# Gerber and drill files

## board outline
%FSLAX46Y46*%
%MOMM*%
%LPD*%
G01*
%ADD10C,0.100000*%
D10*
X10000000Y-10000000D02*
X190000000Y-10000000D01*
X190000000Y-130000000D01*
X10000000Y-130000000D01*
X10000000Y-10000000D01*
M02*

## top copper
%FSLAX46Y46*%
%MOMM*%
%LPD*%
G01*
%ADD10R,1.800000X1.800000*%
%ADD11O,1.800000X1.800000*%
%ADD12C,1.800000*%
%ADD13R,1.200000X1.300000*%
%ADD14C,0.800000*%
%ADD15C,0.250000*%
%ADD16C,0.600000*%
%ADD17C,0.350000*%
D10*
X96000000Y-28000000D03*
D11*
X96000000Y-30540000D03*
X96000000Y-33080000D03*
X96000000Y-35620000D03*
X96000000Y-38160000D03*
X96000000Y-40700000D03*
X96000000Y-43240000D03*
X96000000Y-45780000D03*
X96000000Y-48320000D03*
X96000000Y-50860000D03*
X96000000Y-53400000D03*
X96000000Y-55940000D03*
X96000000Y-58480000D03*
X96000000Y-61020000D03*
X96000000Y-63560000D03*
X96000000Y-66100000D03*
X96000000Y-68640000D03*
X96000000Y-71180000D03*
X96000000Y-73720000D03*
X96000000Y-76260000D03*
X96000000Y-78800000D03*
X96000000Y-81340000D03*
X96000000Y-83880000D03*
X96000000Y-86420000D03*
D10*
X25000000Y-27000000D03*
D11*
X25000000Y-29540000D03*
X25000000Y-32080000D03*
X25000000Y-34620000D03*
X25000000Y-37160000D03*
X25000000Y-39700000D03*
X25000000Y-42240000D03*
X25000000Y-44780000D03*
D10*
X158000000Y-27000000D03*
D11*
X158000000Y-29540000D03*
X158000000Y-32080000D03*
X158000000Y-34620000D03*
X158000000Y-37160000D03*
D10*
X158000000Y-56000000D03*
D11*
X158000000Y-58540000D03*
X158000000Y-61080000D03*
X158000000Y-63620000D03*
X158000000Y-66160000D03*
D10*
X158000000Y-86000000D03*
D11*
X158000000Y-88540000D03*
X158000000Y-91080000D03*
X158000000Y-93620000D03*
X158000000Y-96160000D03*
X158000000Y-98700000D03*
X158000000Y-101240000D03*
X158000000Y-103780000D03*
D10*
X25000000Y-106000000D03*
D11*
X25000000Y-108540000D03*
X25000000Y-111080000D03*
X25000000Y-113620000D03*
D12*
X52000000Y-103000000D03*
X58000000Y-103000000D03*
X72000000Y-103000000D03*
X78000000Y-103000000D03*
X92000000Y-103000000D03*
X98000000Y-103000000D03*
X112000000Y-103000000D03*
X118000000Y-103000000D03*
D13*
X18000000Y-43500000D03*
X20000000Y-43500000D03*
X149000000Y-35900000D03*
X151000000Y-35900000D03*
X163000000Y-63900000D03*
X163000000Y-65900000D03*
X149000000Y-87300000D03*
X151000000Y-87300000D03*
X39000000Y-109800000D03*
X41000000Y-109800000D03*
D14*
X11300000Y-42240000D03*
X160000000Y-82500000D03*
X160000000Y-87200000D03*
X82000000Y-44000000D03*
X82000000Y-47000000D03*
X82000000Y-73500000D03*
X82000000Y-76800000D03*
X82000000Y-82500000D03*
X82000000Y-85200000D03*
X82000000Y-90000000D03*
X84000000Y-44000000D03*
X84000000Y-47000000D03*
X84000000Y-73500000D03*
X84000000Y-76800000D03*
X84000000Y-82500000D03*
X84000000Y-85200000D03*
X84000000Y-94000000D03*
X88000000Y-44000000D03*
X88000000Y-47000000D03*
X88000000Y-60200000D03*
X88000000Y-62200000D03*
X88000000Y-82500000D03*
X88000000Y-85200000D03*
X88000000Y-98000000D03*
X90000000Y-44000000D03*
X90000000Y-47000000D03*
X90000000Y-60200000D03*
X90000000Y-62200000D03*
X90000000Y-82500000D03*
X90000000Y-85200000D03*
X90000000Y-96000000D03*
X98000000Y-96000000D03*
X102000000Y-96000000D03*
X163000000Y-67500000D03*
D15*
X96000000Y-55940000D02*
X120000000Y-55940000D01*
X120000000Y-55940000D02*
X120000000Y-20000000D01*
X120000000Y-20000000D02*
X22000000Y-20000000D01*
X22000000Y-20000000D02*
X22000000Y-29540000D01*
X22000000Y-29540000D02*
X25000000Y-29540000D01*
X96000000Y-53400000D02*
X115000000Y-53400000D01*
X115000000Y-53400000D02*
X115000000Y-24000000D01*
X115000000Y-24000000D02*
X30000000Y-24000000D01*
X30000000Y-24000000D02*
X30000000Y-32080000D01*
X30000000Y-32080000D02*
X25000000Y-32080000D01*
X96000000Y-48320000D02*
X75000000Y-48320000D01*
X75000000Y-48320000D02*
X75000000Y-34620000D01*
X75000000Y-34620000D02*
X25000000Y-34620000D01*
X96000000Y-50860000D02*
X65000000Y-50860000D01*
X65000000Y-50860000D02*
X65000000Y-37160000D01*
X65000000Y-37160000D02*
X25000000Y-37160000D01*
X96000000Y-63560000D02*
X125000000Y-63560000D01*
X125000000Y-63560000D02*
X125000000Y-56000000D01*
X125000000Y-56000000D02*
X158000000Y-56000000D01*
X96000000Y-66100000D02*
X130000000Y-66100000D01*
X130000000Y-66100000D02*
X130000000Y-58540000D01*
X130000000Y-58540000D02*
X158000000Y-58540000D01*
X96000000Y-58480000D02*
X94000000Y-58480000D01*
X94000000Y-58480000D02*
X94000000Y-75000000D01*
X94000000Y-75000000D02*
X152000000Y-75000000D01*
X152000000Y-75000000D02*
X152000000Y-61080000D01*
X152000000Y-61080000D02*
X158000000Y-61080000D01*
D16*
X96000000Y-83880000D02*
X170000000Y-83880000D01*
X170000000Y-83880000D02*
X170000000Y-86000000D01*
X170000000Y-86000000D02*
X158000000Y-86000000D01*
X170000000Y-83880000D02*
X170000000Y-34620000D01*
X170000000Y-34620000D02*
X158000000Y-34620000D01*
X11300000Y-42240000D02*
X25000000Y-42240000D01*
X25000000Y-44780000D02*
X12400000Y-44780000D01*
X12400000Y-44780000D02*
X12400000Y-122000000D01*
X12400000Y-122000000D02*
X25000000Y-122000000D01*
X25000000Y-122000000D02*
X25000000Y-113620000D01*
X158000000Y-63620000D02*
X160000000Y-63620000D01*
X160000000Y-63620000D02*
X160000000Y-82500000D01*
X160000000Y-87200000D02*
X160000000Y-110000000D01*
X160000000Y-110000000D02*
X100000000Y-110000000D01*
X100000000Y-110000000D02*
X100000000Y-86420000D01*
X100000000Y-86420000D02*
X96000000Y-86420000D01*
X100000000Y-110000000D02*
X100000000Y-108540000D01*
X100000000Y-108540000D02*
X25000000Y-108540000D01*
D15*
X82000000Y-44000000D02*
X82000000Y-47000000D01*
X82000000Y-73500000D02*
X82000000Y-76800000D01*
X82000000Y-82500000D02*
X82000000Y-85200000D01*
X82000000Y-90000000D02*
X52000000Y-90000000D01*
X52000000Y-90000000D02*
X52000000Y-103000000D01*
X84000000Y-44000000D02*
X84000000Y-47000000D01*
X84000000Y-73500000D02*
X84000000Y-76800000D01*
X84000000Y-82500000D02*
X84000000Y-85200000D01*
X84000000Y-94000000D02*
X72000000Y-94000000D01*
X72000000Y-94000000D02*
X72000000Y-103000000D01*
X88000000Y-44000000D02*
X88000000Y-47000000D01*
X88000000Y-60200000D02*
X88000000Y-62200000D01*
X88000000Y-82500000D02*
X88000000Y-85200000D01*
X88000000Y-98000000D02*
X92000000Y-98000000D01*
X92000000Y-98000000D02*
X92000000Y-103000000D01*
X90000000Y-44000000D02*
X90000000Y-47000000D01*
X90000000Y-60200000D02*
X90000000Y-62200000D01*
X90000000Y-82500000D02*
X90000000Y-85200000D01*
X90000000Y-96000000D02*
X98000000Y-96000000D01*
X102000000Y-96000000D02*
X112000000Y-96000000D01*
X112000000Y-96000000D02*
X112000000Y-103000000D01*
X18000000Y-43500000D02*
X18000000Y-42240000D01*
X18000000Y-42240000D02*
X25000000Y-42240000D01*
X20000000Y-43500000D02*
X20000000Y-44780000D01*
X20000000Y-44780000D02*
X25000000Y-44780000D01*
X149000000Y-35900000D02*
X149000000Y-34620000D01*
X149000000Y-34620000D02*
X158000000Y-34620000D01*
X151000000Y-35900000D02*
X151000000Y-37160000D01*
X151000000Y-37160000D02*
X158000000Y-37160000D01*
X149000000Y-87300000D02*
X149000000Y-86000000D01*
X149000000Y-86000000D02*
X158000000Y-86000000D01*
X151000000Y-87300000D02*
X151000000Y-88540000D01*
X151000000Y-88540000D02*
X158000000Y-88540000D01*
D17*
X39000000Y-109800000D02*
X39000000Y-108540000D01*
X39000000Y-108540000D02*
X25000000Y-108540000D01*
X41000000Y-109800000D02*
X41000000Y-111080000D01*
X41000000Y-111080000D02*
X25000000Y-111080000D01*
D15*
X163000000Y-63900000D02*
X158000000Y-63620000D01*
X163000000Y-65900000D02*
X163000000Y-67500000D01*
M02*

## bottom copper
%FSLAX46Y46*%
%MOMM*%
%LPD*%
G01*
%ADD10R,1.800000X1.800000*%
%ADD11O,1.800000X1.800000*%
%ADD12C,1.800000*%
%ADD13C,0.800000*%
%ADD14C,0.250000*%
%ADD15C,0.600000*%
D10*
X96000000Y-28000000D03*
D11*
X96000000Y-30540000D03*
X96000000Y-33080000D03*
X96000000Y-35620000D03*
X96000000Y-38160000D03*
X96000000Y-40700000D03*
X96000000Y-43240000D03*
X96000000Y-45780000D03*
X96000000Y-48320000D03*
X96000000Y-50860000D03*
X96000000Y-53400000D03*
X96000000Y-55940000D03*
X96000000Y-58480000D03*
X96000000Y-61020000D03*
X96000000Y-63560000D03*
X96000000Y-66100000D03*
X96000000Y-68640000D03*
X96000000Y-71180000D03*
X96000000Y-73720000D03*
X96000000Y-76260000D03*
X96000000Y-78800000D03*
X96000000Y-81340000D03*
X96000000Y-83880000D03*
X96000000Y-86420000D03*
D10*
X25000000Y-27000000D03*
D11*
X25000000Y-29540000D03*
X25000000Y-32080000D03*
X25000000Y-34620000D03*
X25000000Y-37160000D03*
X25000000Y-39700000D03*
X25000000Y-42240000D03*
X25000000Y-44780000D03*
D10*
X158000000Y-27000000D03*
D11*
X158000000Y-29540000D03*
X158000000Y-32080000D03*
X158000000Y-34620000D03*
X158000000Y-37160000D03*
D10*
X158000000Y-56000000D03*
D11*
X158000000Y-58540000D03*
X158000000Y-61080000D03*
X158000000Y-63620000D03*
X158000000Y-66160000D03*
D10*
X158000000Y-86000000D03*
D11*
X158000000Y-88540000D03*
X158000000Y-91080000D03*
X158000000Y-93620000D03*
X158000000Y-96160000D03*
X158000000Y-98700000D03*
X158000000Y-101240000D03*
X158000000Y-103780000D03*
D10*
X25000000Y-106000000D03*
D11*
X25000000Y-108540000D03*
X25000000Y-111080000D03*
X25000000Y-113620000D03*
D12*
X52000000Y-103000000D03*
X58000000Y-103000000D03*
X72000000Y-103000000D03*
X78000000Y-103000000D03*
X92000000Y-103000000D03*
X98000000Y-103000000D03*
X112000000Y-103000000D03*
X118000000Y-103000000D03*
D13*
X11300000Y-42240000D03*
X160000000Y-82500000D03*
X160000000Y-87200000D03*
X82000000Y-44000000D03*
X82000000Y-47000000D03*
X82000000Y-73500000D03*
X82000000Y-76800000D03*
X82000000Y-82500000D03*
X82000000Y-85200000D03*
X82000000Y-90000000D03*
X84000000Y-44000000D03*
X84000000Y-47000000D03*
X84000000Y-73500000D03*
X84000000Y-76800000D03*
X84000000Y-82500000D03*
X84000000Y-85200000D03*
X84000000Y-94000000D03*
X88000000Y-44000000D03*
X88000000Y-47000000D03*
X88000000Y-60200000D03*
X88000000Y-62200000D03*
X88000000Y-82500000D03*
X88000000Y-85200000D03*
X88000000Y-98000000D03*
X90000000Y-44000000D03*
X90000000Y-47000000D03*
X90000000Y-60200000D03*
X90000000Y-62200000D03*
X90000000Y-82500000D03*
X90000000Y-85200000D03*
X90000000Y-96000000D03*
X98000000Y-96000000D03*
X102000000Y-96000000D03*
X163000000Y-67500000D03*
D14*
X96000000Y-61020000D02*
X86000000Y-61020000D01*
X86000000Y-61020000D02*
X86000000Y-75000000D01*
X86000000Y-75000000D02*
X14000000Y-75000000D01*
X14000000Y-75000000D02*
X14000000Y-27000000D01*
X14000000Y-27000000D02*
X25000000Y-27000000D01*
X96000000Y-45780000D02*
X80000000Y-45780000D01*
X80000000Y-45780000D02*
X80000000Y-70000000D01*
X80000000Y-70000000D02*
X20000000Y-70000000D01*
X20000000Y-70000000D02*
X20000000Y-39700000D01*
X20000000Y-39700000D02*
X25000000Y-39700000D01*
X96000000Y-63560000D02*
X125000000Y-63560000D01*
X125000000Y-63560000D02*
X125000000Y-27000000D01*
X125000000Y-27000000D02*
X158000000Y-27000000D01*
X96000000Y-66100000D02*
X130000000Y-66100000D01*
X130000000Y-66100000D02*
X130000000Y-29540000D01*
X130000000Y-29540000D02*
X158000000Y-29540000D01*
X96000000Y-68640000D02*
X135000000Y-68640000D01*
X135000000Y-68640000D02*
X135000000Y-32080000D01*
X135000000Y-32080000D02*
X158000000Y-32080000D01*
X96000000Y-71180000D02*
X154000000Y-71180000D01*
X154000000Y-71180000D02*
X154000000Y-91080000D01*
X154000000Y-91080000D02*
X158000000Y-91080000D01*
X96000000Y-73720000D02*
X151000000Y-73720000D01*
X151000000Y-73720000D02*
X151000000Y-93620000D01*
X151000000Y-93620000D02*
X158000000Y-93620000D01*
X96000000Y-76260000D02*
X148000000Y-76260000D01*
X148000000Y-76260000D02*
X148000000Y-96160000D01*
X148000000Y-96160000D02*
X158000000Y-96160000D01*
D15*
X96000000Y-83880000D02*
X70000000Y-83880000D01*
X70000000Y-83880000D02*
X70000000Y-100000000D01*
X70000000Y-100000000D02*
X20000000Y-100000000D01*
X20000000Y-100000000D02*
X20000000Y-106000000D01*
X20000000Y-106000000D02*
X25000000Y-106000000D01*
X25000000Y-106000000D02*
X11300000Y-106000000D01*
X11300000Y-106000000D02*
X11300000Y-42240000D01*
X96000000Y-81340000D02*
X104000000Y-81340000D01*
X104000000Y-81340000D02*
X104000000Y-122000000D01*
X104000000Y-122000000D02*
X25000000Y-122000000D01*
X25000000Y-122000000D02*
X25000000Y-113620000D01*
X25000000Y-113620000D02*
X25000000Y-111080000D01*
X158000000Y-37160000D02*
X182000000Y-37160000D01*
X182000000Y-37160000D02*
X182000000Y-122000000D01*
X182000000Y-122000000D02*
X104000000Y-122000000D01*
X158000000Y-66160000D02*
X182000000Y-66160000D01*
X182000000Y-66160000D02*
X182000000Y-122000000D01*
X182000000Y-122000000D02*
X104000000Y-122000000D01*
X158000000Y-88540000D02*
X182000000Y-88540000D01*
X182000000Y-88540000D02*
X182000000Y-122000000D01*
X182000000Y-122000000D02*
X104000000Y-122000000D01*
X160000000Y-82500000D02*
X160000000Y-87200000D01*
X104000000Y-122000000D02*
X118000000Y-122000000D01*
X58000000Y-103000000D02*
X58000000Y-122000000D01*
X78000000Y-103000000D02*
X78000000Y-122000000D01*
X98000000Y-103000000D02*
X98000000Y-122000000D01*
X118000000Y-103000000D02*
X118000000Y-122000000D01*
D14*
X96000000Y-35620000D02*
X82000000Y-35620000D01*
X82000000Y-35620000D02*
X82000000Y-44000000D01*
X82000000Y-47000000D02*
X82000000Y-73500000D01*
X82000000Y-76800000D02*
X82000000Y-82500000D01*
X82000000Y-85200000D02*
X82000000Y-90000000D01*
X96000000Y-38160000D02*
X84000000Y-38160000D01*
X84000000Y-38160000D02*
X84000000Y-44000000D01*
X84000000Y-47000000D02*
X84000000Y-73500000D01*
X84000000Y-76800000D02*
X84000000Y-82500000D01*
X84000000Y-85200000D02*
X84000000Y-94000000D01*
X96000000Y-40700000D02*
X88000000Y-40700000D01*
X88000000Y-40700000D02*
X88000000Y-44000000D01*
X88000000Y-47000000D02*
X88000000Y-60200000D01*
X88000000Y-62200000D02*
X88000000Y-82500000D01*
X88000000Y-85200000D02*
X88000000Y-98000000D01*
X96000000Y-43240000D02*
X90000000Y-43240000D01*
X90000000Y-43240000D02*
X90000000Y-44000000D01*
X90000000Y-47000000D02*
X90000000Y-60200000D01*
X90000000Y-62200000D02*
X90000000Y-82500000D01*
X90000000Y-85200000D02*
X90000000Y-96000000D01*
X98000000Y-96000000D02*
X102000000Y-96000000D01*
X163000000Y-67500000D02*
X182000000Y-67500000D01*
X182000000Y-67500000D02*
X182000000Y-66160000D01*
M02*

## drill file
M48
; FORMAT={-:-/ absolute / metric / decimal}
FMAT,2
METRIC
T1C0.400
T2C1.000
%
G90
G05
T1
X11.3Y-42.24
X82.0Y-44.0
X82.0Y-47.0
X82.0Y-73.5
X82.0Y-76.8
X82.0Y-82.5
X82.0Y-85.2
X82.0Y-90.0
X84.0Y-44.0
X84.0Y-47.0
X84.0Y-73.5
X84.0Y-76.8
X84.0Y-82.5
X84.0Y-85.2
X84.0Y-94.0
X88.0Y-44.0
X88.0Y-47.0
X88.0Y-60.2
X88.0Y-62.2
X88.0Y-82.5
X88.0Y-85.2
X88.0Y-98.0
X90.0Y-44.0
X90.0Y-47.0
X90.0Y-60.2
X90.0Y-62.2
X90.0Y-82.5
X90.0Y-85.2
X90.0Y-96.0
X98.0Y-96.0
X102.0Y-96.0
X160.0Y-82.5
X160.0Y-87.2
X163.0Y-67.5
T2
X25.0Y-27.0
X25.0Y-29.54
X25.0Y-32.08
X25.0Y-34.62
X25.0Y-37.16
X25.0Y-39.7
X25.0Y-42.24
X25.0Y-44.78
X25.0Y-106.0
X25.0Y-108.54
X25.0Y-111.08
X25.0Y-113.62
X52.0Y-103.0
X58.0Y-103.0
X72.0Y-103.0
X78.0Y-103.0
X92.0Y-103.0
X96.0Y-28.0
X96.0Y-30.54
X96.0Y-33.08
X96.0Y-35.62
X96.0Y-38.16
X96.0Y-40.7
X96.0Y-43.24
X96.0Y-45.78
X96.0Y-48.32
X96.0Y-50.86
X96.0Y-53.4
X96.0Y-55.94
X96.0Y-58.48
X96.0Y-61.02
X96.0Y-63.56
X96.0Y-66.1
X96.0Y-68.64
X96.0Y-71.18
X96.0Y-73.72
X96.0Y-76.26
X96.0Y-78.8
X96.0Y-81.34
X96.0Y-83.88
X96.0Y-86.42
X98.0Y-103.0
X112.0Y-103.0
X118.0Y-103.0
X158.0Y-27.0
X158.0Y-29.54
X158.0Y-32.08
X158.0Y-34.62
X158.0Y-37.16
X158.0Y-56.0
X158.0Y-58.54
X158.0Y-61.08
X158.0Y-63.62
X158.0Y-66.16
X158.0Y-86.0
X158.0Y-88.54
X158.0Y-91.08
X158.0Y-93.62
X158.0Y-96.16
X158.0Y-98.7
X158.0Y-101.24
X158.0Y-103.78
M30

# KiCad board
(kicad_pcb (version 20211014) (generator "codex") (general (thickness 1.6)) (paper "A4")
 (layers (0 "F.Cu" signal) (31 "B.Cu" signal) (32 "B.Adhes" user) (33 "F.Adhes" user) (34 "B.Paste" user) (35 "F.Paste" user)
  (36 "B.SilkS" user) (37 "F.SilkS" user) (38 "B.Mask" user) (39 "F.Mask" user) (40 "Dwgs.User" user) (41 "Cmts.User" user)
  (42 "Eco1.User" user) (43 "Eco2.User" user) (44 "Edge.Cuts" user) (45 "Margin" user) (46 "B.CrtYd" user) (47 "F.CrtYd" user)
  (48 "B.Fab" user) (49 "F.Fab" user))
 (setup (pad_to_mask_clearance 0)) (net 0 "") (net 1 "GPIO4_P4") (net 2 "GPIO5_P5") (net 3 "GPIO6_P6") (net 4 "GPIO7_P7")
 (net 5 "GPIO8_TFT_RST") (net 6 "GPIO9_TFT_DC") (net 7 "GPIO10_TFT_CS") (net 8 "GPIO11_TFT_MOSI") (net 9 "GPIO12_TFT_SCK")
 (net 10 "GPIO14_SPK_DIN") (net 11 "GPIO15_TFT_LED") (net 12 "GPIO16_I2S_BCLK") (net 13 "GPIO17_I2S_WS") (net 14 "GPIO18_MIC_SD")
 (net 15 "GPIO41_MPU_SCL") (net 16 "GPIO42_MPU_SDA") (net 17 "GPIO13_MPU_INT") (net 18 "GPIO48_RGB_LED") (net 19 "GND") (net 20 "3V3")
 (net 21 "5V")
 (gr_rect (start 10 10) (end 190 130) (layer "Edge.Cuts") (width 0.1))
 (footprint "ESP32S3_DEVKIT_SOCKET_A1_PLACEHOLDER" (layer "F.Cu") (at 96 28)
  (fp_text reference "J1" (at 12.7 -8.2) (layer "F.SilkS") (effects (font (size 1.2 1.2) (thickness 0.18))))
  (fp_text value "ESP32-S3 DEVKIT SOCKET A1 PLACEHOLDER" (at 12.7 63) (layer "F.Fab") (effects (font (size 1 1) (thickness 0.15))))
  (pad "1" thru_hole rect (at 0 0) (size 1.8 1.8) (drill 1) (layers *.Cu *.Mask))
  (pad "2" thru_hole oval (at 0 2.54) (size 1.8 1.8) (drill 1) (layers *.Cu *.Mask))
  (pad "3" thru_hole oval (at 0 5.08) (size 1.8 1.8) (drill 1) (layers *.Cu *.Mask))
  (pad "4" thru_hole oval (at 0 7.62) (size 1.8 1.8) (drill 1) (layers *.Cu *.Mask) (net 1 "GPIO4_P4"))
  (pad "5" thru_hole oval (at 0 10.16) (size 1.8 1.8) (drill 1) (layers *.Cu *.Mask) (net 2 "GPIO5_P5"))
  (pad "6" thru_hole oval (at 0 12.7) (size 1.8 1.8) (drill 1) (layers *.Cu *.Mask) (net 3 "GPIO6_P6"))
  (pad "7" thru_hole oval (at 0 15.24) (size 1.8 1.8) (drill 1) (layers *.Cu *.Mask) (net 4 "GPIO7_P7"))
  (pad "8" thru_hole oval (at 0 17.78) (size 1.8 1.8) (drill 1) (layers *.Cu *.Mask) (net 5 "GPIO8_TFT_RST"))
  (pad "9" thru_hole oval (at 0 20.32) (size 1.8 1.8) (drill 1) (layers *.Cu *.Mask) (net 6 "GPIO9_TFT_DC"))
  (pad "10" thru_hole oval (at 0 22.86) (size 1.8 1.8) (drill 1) (layers *.Cu *.Mask) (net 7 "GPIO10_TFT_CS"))
  (pad "11" thru_hole oval (at 0 25.4) (size 1.8 1.8) (drill 1) (layers *.Cu *.Mask) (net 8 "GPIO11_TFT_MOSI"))
  (pad "12" thru_hole oval (at 0 27.94) (size 1.8 1.8) (drill 1) (layers *.Cu *.Mask) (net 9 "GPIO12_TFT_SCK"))
  (pad "13" thru_hole oval (at 0 30.48) (size 1.8 1.8) (drill 1) (layers *.Cu *.Mask) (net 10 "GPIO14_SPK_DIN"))
  (pad "14" thru_hole oval (at 0 33.02) (size 1.8 1.8) (drill 1) (layers *.Cu *.Mask) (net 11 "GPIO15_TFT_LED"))
  (pad "15" thru_hole oval (at 0 35.56) (size 1.8 1.8) (drill 1) (layers *.Cu *.Mask) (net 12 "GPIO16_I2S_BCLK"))
  (pad "16" thru_hole oval (at 0 38.1) (size 1.8 1.8) (drill 1) (layers *.Cu *.Mask) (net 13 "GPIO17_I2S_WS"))
  (pad "17" thru_hole oval (at 0 40.64) (size 1.8 1.8) (drill 1) (layers *.Cu *.Mask) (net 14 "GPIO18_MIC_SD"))
  (pad "18" thru_hole oval (at 0 43.18) (size 1.8 1.8) (drill 1) (layers *.Cu *.Mask) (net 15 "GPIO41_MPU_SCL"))
  (pad "19" thru_hole oval (at 0 45.72) (size 1.8 1.8) (drill 1) (layers *.Cu *.Mask) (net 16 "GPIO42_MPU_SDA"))
  (pad "20" thru_hole oval (at 0 48.26) (size 1.8 1.8) (drill 1) (layers *.Cu *.Mask) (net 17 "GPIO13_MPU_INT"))
  (pad "21" thru_hole oval (at 0 50.8) (size 1.8 1.8) (drill 1) (layers *.Cu *.Mask) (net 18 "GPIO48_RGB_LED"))
  (pad "22" thru_hole oval (at 0 53.34) (size 1.8 1.8) (drill 1) (layers *.Cu *.Mask) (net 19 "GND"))
  (pad "23" thru_hole oval (at 0 55.88) (size 1.8 1.8) (drill 1) (layers *.Cu *.Mask) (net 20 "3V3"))
  (pad "24" thru_hole oval (at 0 58.42) (size 1.8 1.8) (drill 1) (layers *.Cu *.Mask) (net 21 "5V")))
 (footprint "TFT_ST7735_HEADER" (layer "F.Cu") (at 25 27)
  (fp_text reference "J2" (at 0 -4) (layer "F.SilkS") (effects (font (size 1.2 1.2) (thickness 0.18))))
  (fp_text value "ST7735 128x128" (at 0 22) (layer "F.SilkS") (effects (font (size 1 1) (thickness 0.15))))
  (pad "1" thru_hole rect (at 0 0) (size 1.8 1.8) (drill 1) (layers *.Cu *.Mask) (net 11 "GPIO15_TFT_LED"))
  (pad "2" thru_hole oval (at 0 2.54) (size 1.8 1.8) (drill 1) (layers *.Cu *.Mask) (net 9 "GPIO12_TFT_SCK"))
  (pad "3" thru_hole oval (at 0 5.08) (size 1.8 1.8) (drill 1) (layers *.Cu *.Mask) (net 8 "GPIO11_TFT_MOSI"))
  (pad "4" thru_hole oval (at 0 7.62) (size 1.8 1.8) (drill 1) (layers *.Cu *.Mask) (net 6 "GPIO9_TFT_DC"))
  (pad "5" thru_hole oval (at 0 10.16) (size 1.8 1.8) (drill 1) (layers *.Cu *.Mask) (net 7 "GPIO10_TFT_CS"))
  (pad "6" thru_hole oval (at 0 12.7) (size 1.8 1.8) (drill 1) (layers *.Cu *.Mask) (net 5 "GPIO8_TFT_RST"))
  (pad "7" thru_hole oval (at 0 15.24) (size 1.8 1.8) (drill 1) (layers *.Cu *.Mask) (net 20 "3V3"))
  (pad "8" thru_hole oval (at 0 17.78) (size 1.8 1.8) (drill 1) (layers *.Cu *.Mask) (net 19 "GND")))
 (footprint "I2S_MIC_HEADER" (layer "F.Cu") (at 158 27)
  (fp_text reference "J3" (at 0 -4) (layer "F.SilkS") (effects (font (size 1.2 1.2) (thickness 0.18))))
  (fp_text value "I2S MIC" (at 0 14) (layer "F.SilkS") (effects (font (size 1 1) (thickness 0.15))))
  (pad "1" thru_hole rect (at 0 0) (size 1.8 1.8) (drill 1) (layers *.Cu *.Mask) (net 12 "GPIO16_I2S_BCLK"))
  (pad "2" thru_hole oval (at 0 2.54) (size 1.8 1.8) (drill 1) (layers *.Cu *.Mask) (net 13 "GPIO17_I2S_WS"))
  (pad "3" thru_hole oval (at 0 5.08) (size 1.8 1.8) (drill 1) (layers *.Cu *.Mask) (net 14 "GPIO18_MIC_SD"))
  (pad "4" thru_hole oval (at 0 7.62) (size 1.8 1.8) (drill 1) (layers *.Cu *.Mask) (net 20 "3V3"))
  (pad "5" thru_hole oval (at 0 10.16) (size 1.8 1.8) (drill 1) (layers *.Cu *.Mask) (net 19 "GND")))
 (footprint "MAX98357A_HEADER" (layer "F.Cu") (at 158 56)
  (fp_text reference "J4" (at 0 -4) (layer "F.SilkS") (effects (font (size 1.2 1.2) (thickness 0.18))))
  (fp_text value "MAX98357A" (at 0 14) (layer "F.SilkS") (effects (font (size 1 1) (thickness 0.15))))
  (pad "1" thru_hole rect (at 0 0) (size 1.8 1.8) (drill 1) (layers *.Cu *.Mask) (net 12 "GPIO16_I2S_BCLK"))
  (pad "2" thru_hole oval (at 0 2.54) (size 1.8 1.8) (drill 1) (layers *.Cu *.Mask) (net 13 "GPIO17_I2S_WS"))
  (pad "3" thru_hole oval (at 0 5.08) (size 1.8 1.8) (drill 1) (layers *.Cu *.Mask) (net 10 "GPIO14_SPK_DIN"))
  (pad "4" thru_hole oval (at 0 7.62) (size 1.8 1.8) (drill 1) (layers *.Cu *.Mask) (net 21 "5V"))
  (pad "5" thru_hole oval (at 0 10.16) (size 1.8 1.8) (drill 1) (layers *.Cu *.Mask) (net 19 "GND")))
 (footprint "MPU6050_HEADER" (layer "F.Cu") (at 158 86)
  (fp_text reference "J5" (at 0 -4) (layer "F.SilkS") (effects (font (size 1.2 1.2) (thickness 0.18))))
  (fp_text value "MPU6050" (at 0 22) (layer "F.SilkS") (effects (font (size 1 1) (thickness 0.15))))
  (pad "1" thru_hole rect (at 0 0) (size 1.8 1.8) (drill 1) (layers *.Cu *.Mask) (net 20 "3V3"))
  (pad "2" thru_hole oval (at 0 2.54) (size 1.8 1.8) (drill 1) (layers *.Cu *.Mask) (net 19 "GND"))
  (pad "3" thru_hole oval (at 0 5.08) (size 1.8 1.8) (drill 1) (layers *.Cu *.Mask) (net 15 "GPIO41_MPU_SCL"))
  (pad "4" thru_hole oval (at 0 7.62) (size 1.8 1.8) (drill 1) (layers *.Cu *.Mask) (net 16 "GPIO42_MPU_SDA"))
  (pad "5" thru_hole oval (at 0 10.16) (size 1.8 1.8) (drill 1) (layers *.Cu *.Mask) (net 17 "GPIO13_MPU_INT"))
  (pad "6" thru_hole oval (at 0 12.7) (size 1.8 1.8) (drill 1) (layers *.Cu *.Mask))
  (pad "7" thru_hole oval (at 0 15.24) (size 1.8 1.8) (drill 1) (layers *.Cu *.Mask))
  (pad "8" thru_hole oval (at 0 17.78) (size 1.8 1.8) (drill 1) (layers *.Cu *.Mask)))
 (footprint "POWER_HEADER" (layer "F.Cu") (at 25 106)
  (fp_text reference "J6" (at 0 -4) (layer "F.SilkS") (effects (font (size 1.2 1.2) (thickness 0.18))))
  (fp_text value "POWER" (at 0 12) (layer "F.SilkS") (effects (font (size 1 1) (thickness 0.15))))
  (pad "1" thru_hole rect (at 0 0) (size 1.8 1.8) (drill 1) (layers *.Cu *.Mask) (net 20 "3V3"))
  (pad "2" thru_hole oval (at 0 2.54) (size 1.8 1.8) (drill 1) (layers *.Cu *.Mask) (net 21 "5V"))
  (pad "3" thru_hole oval (at 0 5.08) (size 1.8 1.8) (drill 1) (layers *.Cu *.Mask) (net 19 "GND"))
  (pad "4" thru_hole oval (at 0 7.62) (size 1.8 1.8) (drill 1) (layers *.Cu *.Mask) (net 19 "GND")))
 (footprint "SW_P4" (layer "F.Cu") (at 55 103)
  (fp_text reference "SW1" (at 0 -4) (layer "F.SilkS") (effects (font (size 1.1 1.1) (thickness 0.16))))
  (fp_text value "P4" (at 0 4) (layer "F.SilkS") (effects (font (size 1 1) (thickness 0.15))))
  (pad "1" thru_hole circle (at -3 0) (size 1.8 1.8) (drill 1) (layers *.Cu *.Mask) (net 1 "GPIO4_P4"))
  (pad "2" thru_hole circle (at 3 0) (size 1.8 1.8) (drill 1) (layers *.Cu *.Mask) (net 19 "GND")))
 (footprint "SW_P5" (layer "F.Cu") (at 75 103)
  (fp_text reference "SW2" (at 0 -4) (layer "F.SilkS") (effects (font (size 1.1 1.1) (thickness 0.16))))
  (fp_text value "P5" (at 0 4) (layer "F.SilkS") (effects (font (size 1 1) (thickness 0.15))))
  (pad "1" thru_hole circle (at -3 0) (size 1.8 1.8) (drill 1) (layers *.Cu *.Mask) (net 2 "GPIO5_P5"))
  (pad "2" thru_hole circle (at 3 0) (size 1.8 1.8) (drill 1) (layers *.Cu *.Mask) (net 19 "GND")))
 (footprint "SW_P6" (layer "F.Cu") (at 95 103)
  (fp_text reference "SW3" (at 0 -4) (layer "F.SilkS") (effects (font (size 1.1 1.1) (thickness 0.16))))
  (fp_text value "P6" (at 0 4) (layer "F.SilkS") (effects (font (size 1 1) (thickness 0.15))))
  (pad "1" thru_hole circle (at -3 0) (size 1.8 1.8) (drill 1) (layers *.Cu *.Mask) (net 3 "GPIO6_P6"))
  (pad "2" thru_hole circle (at 3 0) (size 1.8 1.8) (drill 1) (layers *.Cu *.Mask) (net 19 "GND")))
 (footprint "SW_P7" (layer "F.Cu") (at 115 103)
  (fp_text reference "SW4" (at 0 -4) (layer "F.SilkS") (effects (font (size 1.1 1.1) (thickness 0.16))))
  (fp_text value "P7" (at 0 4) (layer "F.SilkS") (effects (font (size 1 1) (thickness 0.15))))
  (pad "1" thru_hole circle (at -3 0) (size 1.8 1.8) (drill 1) (layers *.Cu *.Mask) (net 4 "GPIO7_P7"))
  (pad "2" thru_hole circle (at 3 0) (size 1.8 1.8) (drill 1) (layers *.Cu *.Mask) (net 19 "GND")))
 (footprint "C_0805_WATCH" (layer "F.Cu") (at 19.00 43.50)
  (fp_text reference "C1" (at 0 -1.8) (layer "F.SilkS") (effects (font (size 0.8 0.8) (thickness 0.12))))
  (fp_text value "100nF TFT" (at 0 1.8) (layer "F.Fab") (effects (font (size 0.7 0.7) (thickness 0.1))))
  (pad "1" smd rect (at -1.00 0) (size 1.20 1.30) (layers "F.Cu" "F.Paste" "F.Mask") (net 20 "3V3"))
  (pad "2" smd rect (at 1.00 0) (size 1.20 1.30) (layers "F.Cu" "F.Paste" "F.Mask") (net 19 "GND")))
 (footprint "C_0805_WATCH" (layer "F.Cu") (at 150.00 35.90)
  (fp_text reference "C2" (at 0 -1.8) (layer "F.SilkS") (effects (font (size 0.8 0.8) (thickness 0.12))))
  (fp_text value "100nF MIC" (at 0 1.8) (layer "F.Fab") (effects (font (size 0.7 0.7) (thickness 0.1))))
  (pad "1" smd rect (at -1.00 0) (size 1.20 1.30) (layers "F.Cu" "F.Paste" "F.Mask") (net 20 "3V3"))
  (pad "2" smd rect (at 1.00 0) (size 1.20 1.30) (layers "F.Cu" "F.Paste" "F.Mask") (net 19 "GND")))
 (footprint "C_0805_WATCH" (layer "F.Cu") (at 163.00 64.90 270)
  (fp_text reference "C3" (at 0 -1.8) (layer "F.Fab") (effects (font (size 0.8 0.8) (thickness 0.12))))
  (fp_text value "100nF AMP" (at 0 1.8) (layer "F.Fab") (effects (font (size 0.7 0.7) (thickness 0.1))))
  (pad "1" smd rect (at -1.00 0) (size 1.20 1.30) (layers "F.Cu" "F.Paste" "F.Mask") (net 21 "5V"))
  (pad "2" smd rect (at 1.00 0) (size 1.20 1.30) (layers "F.Cu" "F.Paste" "F.Mask") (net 19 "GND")))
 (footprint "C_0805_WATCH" (layer "F.Cu") (at 150.00 87.30)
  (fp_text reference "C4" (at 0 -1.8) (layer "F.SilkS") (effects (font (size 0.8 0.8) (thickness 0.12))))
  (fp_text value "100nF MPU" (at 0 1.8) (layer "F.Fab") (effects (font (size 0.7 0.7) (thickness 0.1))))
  (pad "1" smd rect (at -1.00 0) (size 1.20 1.30) (layers "F.Cu" "F.Paste" "F.Mask") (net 20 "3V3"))
  (pad "2" smd rect (at 1.00 0) (size 1.20 1.30) (layers "F.Cu" "F.Paste" "F.Mask") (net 19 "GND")))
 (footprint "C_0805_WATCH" (layer "F.Cu") (at 40.00 109.80)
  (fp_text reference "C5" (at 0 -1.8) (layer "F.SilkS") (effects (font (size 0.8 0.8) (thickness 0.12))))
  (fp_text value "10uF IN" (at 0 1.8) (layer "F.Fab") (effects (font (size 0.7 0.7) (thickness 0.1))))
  (pad "1" smd rect (at -1.00 0) (size 1.20 1.30) (layers "F.Cu" "F.Paste" "F.Mask") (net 21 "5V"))
  (pad "2" smd rect (at 1.00 0) (size 1.20 1.30) (layers "F.Cu" "F.Paste" "F.Mask") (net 19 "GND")))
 (segment (start 96.00 61.02) (end 86.00 61.02) (width 0.25) (layer "B.Cu") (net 11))
 (segment (start 86.00 61.02) (end 86.00 75.00) (width 0.25) (layer "B.Cu") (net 11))
 (segment (start 86.00 75.00) (end 14.00 75.00) (width 0.25) (layer "B.Cu") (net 11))
 (segment (start 14.00 75.00) (end 14.00 27.00) (width 0.25) (layer "B.Cu") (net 11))
 (segment (start 14.00 27.00) (end 25.00 27.00) (width 0.25) (layer "B.Cu") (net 11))
 (segment (start 96.00 55.94) (end 120.00 55.94) (width 0.25) (layer "F.Cu") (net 9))
 (segment (start 120.00 55.94) (end 120.00 20.00) (width 0.25) (layer "F.Cu") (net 9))
 (segment (start 120.00 20.00) (end 22.00 20.00) (width 0.25) (layer "F.Cu") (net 9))
 (segment (start 22.00 20.00) (end 22.00 29.54) (width 0.25) (layer "F.Cu") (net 9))
 (segment (start 22.00 29.54) (end 25.00 29.54) (width 0.25) (layer "F.Cu") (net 9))
 (segment (start 96.00 53.40) (end 115.00 53.40) (width 0.25) (layer "F.Cu") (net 8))
 (segment (start 115.00 53.40) (end 115.00 24.00) (width 0.25) (layer "F.Cu") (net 8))
 (segment (start 115.00 24.00) (end 30.00 24.00) (width 0.25) (layer "F.Cu") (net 8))
 (segment (start 30.00 24.00) (end 30.00 32.08) (width 0.25) (layer "F.Cu") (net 8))
 (segment (start 30.00 32.08) (end 25.00 32.08) (width 0.25) (layer "F.Cu") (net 8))
 (segment (start 96.00 48.32) (end 75.00 48.32) (width 0.25) (layer "F.Cu") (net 6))
 (segment (start 75.00 48.32) (end 75.00 34.62) (width 0.25) (layer "F.Cu") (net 6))
 (segment (start 75.00 34.62) (end 25.00 34.62) (width 0.25) (layer "F.Cu") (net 6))
 (segment (start 96.00 50.86) (end 65.00 50.86) (width 0.25) (layer "F.Cu") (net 7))
 (segment (start 65.00 50.86) (end 65.00 37.16) (width 0.25) (layer "F.Cu") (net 7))
 (segment (start 65.00 37.16) (end 25.00 37.16) (width 0.25) (layer "F.Cu") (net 7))
 (segment (start 96.00 45.78) (end 80.00 45.78) (width 0.25) (layer "B.Cu") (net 5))
 (segment (start 80.00 45.78) (end 80.00 70.00) (width 0.25) (layer "B.Cu") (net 5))
 (segment (start 80.00 70.00) (end 20.00 70.00) (width 0.25) (layer "B.Cu") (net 5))
 (segment (start 20.00 70.00) (end 20.00 39.70) (width 0.25) (layer "B.Cu") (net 5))
 (segment (start 20.00 39.70) (end 25.00 39.70) (width 0.25) (layer "B.Cu") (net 5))
 (segment (start 96.00 63.56) (end 125.00 63.56) (width 0.25) (layer "B.Cu") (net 12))
 (segment (start 125.00 63.56) (end 125.00 27.00) (width 0.25) (layer "B.Cu") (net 12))
 (segment (start 125.00 27.00) (end 158.00 27.00) (width 0.25) (layer "B.Cu") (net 12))
 (segment (start 96.00 66.10) (end 130.00 66.10) (width 0.25) (layer "B.Cu") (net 13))
 (segment (start 130.00 66.10) (end 130.00 29.54) (width 0.25) (layer "B.Cu") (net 13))
 (segment (start 130.00 29.54) (end 158.00 29.54) (width 0.25) (layer "B.Cu") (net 13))
 (segment (start 96.00 68.64) (end 135.00 68.64) (width 0.25) (layer "B.Cu") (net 14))
 (segment (start 135.00 68.64) (end 135.00 32.08) (width 0.25) (layer "B.Cu") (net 14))
 (segment (start 135.00 32.08) (end 158.00 32.08) (width 0.25) (layer "B.Cu") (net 14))
 (segment (start 96.00 63.56) (end 125.00 63.56) (width 0.25) (layer "F.Cu") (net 12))
 (segment (start 125.00 63.56) (end 125.00 56.00) (width 0.25) (layer "F.Cu") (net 12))
 (segment (start 125.00 56.00) (end 158.00 56.00) (width 0.25) (layer "F.Cu") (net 12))
 (segment (start 96.00 66.10) (end 130.00 66.10) (width 0.25) (layer "F.Cu") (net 13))
 (segment (start 130.00 66.10) (end 130.00 58.54) (width 0.25) (layer "F.Cu") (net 13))
 (segment (start 130.00 58.54) (end 158.00 58.54) (width 0.25) (layer "F.Cu") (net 13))
 (segment (start 96.00 58.48) (end 94.00 58.48) (width 0.25) (layer "F.Cu") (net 10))
 (segment (start 94.00 58.48) (end 94.00 75.00) (width 0.25) (layer "F.Cu") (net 10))
 (segment (start 94.00 75.00) (end 152.00 75.00) (width 0.25) (layer "F.Cu") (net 10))
 (segment (start 152.00 75.00) (end 152.00 61.08) (width 0.25) (layer "F.Cu") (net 10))
 (segment (start 152.00 61.08) (end 158.00 61.08) (width 0.25) (layer "F.Cu") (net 10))
 (segment (start 96.00 71.18) (end 154.00 71.18) (width 0.25) (layer "B.Cu") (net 15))
 (segment (start 154.00 71.18) (end 154.00 91.08) (width 0.25) (layer "B.Cu") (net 15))
 (segment (start 154.00 91.08) (end 158.00 91.08) (width 0.25) (layer "B.Cu") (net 15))
 (segment (start 96.00 73.72) (end 151.00 73.72) (width 0.25) (layer "B.Cu") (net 16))
 (segment (start 151.00 73.72) (end 151.00 93.62) (width 0.25) (layer "B.Cu") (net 16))
 (segment (start 151.00 93.62) (end 158.00 93.62) (width 0.25) (layer "B.Cu") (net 16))
 (segment (start 96.00 76.26) (end 148.00 76.26) (width 0.25) (layer "B.Cu") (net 17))
 (segment (start 148.00 76.26) (end 148.00 96.16) (width 0.25) (layer "B.Cu") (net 17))
 (segment (start 148.00 96.16) (end 158.00 96.16) (width 0.25) (layer "B.Cu") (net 17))
 (segment (start 96.00 83.88) (end 170.00 83.88) (width 0.60) (layer "F.Cu") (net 20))
 (segment (start 170.00 83.88) (end 170.00 86.00) (width 0.60) (layer "F.Cu") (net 20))
 (segment (start 170.00 86.00) (end 158.00 86.00) (width 0.60) (layer "F.Cu") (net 20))
 (segment (start 170.00 83.88) (end 170.00 34.62) (width 0.60) (layer "F.Cu") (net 20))
 (segment (start 170.00 34.62) (end 158.00 34.62) (width 0.60) (layer "F.Cu") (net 20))
 (segment (start 96.00 83.88) (end 70.00 83.88) (width 0.60) (layer "B.Cu") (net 20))
 (segment (start 70.00 83.88) (end 70.00 100.00) (width 0.60) (layer "B.Cu") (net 20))
 (segment (start 70.00 100.00) (end 20.00 100.00) (width 0.60) (layer "B.Cu") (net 20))
 (segment (start 20.00 100.00) (end 20.00 106.00) (width 0.60) (layer "B.Cu") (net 20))
 (segment (start 20.00 106.00) (end 25.00 106.00) (width 0.60) (layer "B.Cu") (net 20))
 (segment (start 25.00 106.00) (end 11.30 106.00) (width 0.60) (layer "B.Cu") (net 20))
 (segment (start 11.30 106.00) (end 11.30 42.24) (width 0.60) (layer "B.Cu") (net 20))
 (via (at 11.30 42.24) (size 0.80) (drill 0.40) (layers "F.Cu" "B.Cu") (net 20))
 (segment (start 11.30 42.24) (end 25.00 42.24) (width 0.60) (layer "F.Cu") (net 20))
 (segment (start 96.00 81.34) (end 104.00 81.34) (width 0.60) (layer "B.Cu") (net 19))
 (segment (start 104.00 81.34) (end 104.00 122.00) (width 0.60) (layer "B.Cu") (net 19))
 (segment (start 104.00 122.00) (end 25.00 122.00) (width 0.60) (layer "B.Cu") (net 19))
 (segment (start 25.00 122.00) (end 25.00 113.62) (width 0.60) (layer "B.Cu") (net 19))
 (segment (start 25.00 113.62) (end 25.00 111.08) (width 0.60) (layer "B.Cu") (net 19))
 (segment (start 25.00 44.78) (end 12.40 44.78) (width 0.60) (layer "F.Cu") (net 19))
 (segment (start 12.40 44.78) (end 12.40 122.00) (width 0.60) (layer "F.Cu") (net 19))
 (segment (start 12.40 122.00) (end 25.00 122.00) (width 0.60) (layer "F.Cu") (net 19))
 (segment (start 25.00 122.00) (end 25.00 113.62) (width 0.60) (layer "F.Cu") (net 19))
 (segment (start 158.00 37.16) (end 182.00 37.16) (width 0.60) (layer "B.Cu") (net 19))
 (segment (start 182.00 37.16) (end 182.00 122.00) (width 0.60) (layer "B.Cu") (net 19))
 (segment (start 182.00 122.00) (end 104.00 122.00) (width 0.60) (layer "B.Cu") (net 19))
 (segment (start 158.00 66.16) (end 182.00 66.16) (width 0.60) (layer "B.Cu") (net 19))
 (segment (start 182.00 66.16) (end 182.00 122.00) (width 0.60) (layer "B.Cu") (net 19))
 (segment (start 182.00 122.00) (end 104.00 122.00) (width 0.60) (layer "B.Cu") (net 19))
 (segment (start 158.00 88.54) (end 182.00 88.54) (width 0.60) (layer "B.Cu") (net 19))
 (segment (start 182.00 88.54) (end 182.00 122.00) (width 0.60) (layer "B.Cu") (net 19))
 (segment (start 182.00 122.00) (end 104.00 122.00) (width 0.60) (layer "B.Cu") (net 19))
 (segment (start 158.00 63.62) (end 160.00 63.62) (width 0.60) (layer "F.Cu") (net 21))
 (segment (start 160.00 63.62) (end 160.00 82.50) (width 0.60) (layer "F.Cu") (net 21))
 (via (at 160.00 82.50) (size 0.80) (drill 0.40) (layers "F.Cu" "B.Cu") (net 21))
 (segment (start 160.00 82.50) (end 160.00 87.20) (width 0.60) (layer "B.Cu") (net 21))
 (via (at 160.00 87.20) (size 0.80) (drill 0.40) (layers "F.Cu" "B.Cu") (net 21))
 (segment (start 160.00 87.20) (end 160.00 110.00) (width 0.60) (layer "F.Cu") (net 21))
 (segment (start 160.00 110.00) (end 100.00 110.00) (width 0.60) (layer "F.Cu") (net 21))
 (segment (start 100.00 110.00) (end 100.00 86.42) (width 0.60) (layer "F.Cu") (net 21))
 (segment (start 100.00 86.42) (end 96.00 86.42) (width 0.60) (layer "F.Cu") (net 21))
 (segment (start 100.00 110.00) (end 100.00 108.54) (width 0.60) (layer "F.Cu") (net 21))
 (segment (start 100.00 108.54) (end 25.00 108.54) (width 0.60) (layer "F.Cu") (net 21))
 (segment (start 104.00 122.00) (end 118.00 122.00) (width 0.60) (layer "B.Cu") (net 19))
 (segment (start 58.00 103.00) (end 58.00 122.00) (width 0.60) (layer "B.Cu") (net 19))
 (segment (start 78.00 103.00) (end 78.00 122.00) (width 0.60) (layer "B.Cu") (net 19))
 (segment (start 98.00 103.00) (end 98.00 122.00) (width 0.60) (layer "B.Cu") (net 19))
 (segment (start 118.00 103.00) (end 118.00 122.00) (width 0.60) (layer "B.Cu") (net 19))
 (segment (start 96.00 35.62) (end 82.00 35.62) (width 0.25) (layer "B.Cu") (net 1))
 (segment (start 82.00 35.62) (end 82.00 44.00) (width 0.25) (layer "B.Cu") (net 1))
 (via (at 82.00 44.00) (size 0.80) (drill 0.40) (layers "F.Cu" "B.Cu") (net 1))
 (segment (start 82.00 44.00) (end 82.00 47.00) (width 0.25) (layer "F.Cu") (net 1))
 (via (at 82.00 47.00) (size 0.80) (drill 0.40) (layers "F.Cu" "B.Cu") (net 1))
 (segment (start 82.00 47.00) (end 82.00 73.50) (width 0.25) (layer "B.Cu") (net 1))
 (via (at 82.00 73.50) (size 0.80) (drill 0.40) (layers "F.Cu" "B.Cu") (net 1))
 (segment (start 82.00 73.50) (end 82.00 76.80) (width 0.25) (layer "F.Cu") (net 1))
 (via (at 82.00 76.80) (size 0.80) (drill 0.40) (layers "F.Cu" "B.Cu") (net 1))
 (segment (start 82.00 76.80) (end 82.00 82.50) (width 0.25) (layer "B.Cu") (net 1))
 (via (at 82.00 82.50) (size 0.80) (drill 0.40) (layers "F.Cu" "B.Cu") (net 1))
 (segment (start 82.00 82.50) (end 82.00 85.20) (width 0.25) (layer "F.Cu") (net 1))
 (via (at 82.00 85.20) (size 0.80) (drill 0.40) (layers "F.Cu" "B.Cu") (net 1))
 (segment (start 82.00 85.20) (end 82.00 90.00) (width 0.25) (layer "B.Cu") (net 1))
 (via (at 82.00 90.00) (size 0.80) (drill 0.40) (layers "F.Cu" "B.Cu") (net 1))
 (segment (start 82.00 90.00) (end 52.00 90.00) (width 0.25) (layer "F.Cu") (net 1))
 (segment (start 52.00 90.00) (end 52.00 103.00) (width 0.25) (layer "F.Cu") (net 1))
 (segment (start 96.00 38.16) (end 84.00 38.16) (width 0.25) (layer "B.Cu") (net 2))
 (segment (start 84.00 38.16) (end 84.00 44.00) (width 0.25) (layer "B.Cu") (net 2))
 (via (at 84.00 44.00) (size 0.80) (drill 0.40) (layers "F.Cu" "B.Cu") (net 2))
 (segment (start 84.00 44.00) (end 84.00 47.00) (width 0.25) (layer "F.Cu") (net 2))
 (via (at 84.00 47.00) (size 0.80) (drill 0.40) (layers "F.Cu" "B.Cu") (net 2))
 (segment (start 84.00 47.00) (end 84.00 73.50) (width 0.25) (layer "B.Cu") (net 2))
 (via (at 84.00 73.50) (size 0.80) (drill 0.40) (layers "F.Cu" "B.Cu") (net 2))
 (segment (start 84.00 73.50) (end 84.00 76.80) (width 0.25) (layer "F.Cu") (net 2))
 (via (at 84.00 76.80) (size 0.80) (drill 0.40) (layers "F.Cu" "B.Cu") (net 2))
 (segment (start 84.00 76.80) (end 84.00 82.50) (width 0.25) (layer "B.Cu") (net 2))
 (via (at 84.00 82.50) (size 0.80) (drill 0.40) (layers "F.Cu" "B.Cu") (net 2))
 (segment (start 84.00 82.50) (end 84.00 85.20) (width 0.25) (layer "F.Cu") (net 2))
 (via (at 84.00 85.20) (size 0.80) (drill 0.40) (layers "F.Cu" "B.Cu") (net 2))
 (segment (start 84.00 85.20) (end 84.00 94.00) (width 0.25) (layer "B.Cu") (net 2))
 (via (at 84.00 94.00) (size 0.80) (drill 0.40) (layers "F.Cu" "B.Cu") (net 2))
 (segment (start 84.00 94.00) (end 72.00 94.00) (width 0.25) (layer "F.Cu") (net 2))
 (segment (start 72.00 94.00) (end 72.00 103.00) (width 0.25) (layer "F.Cu") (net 2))
 (segment (start 96.00 40.70) (end 88.00 40.70) (width 0.25) (layer "B.Cu") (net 3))
 (segment (start 88.00 40.70) (end 88.00 44.00) (width 0.25) (layer "B.Cu") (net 3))
 (via (at 88.00 44.00) (size 0.80) (drill 0.40) (layers "F.Cu" "B.Cu") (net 3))
 (segment (start 88.00 44.00) (end 88.00 47.00) (width 0.25) (layer "F.Cu") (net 3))
 (via (at 88.00 47.00) (size 0.80) (drill 0.40) (layers "F.Cu" "B.Cu") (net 3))
 (segment (start 88.00 47.00) (end 88.00 60.20) (width 0.25) (layer "B.Cu") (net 3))
 (via (at 88.00 60.20) (size 0.80) (drill 0.40) (layers "F.Cu" "B.Cu") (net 3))
 (segment (start 88.00 60.20) (end 88.00 62.20) (width 0.25) (layer "F.Cu") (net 3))
 (via (at 88.00 62.20) (size 0.80) (drill 0.40) (layers "F.Cu" "B.Cu") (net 3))
 (segment (start 88.00 62.20) (end 88.00 82.50) (width 0.25) (layer "B.Cu") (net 3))
 (via (at 88.00 82.50) (size 0.80) (drill 0.40) (layers "F.Cu" "B.Cu") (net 3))
 (segment (start 88.00 82.50) (end 88.00 85.20) (width 0.25) (layer "F.Cu") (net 3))
 (via (at 88.00 85.20) (size 0.80) (drill 0.40) (layers "F.Cu" "B.Cu") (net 3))
 (segment (start 88.00 85.20) (end 88.00 98.00) (width 0.25) (layer "B.Cu") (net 3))
 (via (at 88.00 98.00) (size 0.80) (drill 0.40) (layers "F.Cu" "B.Cu") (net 3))
 (segment (start 88.00 98.00) (end 92.00 98.00) (width 0.25) (layer "F.Cu") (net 3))
 (segment (start 92.00 98.00) (end 92.00 103.00) (width 0.25) (layer "F.Cu") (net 3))
 (segment (start 96.00 43.24) (end 90.00 43.24) (width 0.25) (layer "B.Cu") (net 4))
 (segment (start 90.00 43.24) (end 90.00 44.00) (width 0.25) (layer "B.Cu") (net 4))
 (via (at 90.00 44.00) (size 0.80) (drill 0.40) (layers "F.Cu" "B.Cu") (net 4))
 (segment (start 90.00 44.00) (end 90.00 47.00) (width 0.25) (layer "F.Cu") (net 4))
 (via (at 90.00 47.00) (size 0.80) (drill 0.40) (layers "F.Cu" "B.Cu") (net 4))
 (segment (start 90.00 47.00) (end 90.00 60.20) (width 0.25) (layer "B.Cu") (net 4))
 (via (at 90.00 60.20) (size 0.80) (drill 0.40) (layers "F.Cu" "B.Cu") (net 4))
 (segment (start 90.00 60.20) (end 90.00 62.20) (width 0.25) (layer "F.Cu") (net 4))
 (via (at 90.00 62.20) (size 0.80) (drill 0.40) (layers "F.Cu" "B.Cu") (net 4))
 (segment (start 90.00 62.20) (end 90.00 82.50) (width 0.25) (layer "B.Cu") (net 4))
 (via (at 90.00 82.50) (size 0.80) (drill 0.40) (layers "F.Cu" "B.Cu") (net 4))
 (segment (start 90.00 82.50) (end 90.00 85.20) (width 0.25) (layer "F.Cu") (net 4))
 (via (at 90.00 85.20) (size 0.80) (drill 0.40) (layers "F.Cu" "B.Cu") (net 4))
 (segment (start 90.00 85.20) (end 90.00 96.00) (width 0.25) (layer "B.Cu") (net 4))
 (via (at 90.00 96.00) (size 0.80) (drill 0.40) (layers "F.Cu" "B.Cu") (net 4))
 (segment (start 90.00 96.00) (end 98.00 96.00) (width 0.25) (layer "F.Cu") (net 4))
 (via (at 98.00 96.00) (size 0.80) (drill 0.40) (layers "F.Cu" "B.Cu") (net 4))
 (segment (start 98.00 96.00) (end 102.00 96.00) (width 0.25) (layer "B.Cu") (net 4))
 (via (at 102.00 96.00) (size 0.80) (drill 0.40) (layers "F.Cu" "B.Cu") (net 4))
 (segment (start 102.00 96.00) (end 112.00 96.00) (width 0.25) (layer "F.Cu") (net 4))
 (segment (start 112.00 96.00) (end 112.00 103.00) (width 0.25) (layer "F.Cu") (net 4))
 (segment (start 18.00 43.50) (end 18.00 42.24) (width 0.25) (layer "F.Cu") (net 20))
 (segment (start 18.00 42.24) (end 25.00 42.24) (width 0.25) (layer "F.Cu") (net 20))
 (segment (start 20.00 43.50) (end 20.00 44.78) (width 0.25) (layer "F.Cu") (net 19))
 (segment (start 20.00 44.78) (end 25.00 44.78) (width 0.25) (layer "F.Cu") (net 19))
 (segment (start 149.00 35.90) (end 149.00 34.62) (width 0.25) (layer "F.Cu") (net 20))
 (segment (start 149.00 34.62) (end 158.00 34.62) (width 0.25) (layer "F.Cu") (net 20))
 (segment (start 151.00 35.90) (end 151.00 37.16) (width 0.25) (layer "F.Cu") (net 19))
 (segment (start 151.00 37.16) (end 158.00 37.16) (width 0.25) (layer "F.Cu") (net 19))
 (segment (start 149.00 87.30) (end 149.00 86.00) (width 0.25) (layer "F.Cu") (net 20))
 (segment (start 149.00 86.00) (end 158.00 86.00) (width 0.25) (layer "F.Cu") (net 20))
 (segment (start 151.00 87.30) (end 151.00 88.54) (width 0.25) (layer "F.Cu") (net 19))
 (segment (start 151.00 88.54) (end 158.00 88.54) (width 0.25) (layer "F.Cu") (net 19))
 (segment (start 39.00 109.80) (end 39.00 108.54) (width 0.35) (layer "F.Cu") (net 21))
 (segment (start 39.00 108.54) (end 25.00 108.54) (width 0.35) (layer "F.Cu") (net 21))
 (segment (start 41.00 109.80) (end 41.00 111.08) (width 0.35) (layer "F.Cu") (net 19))
 (segment (start 41.00 111.08) (end 25.00 111.08) (width 0.35) (layer "F.Cu") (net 19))
 (segment (start 163.00 63.90) (end 158.00 63.62) (width 0.25) (layer "F.Cu") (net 21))
 (segment (start 163.00 65.90) (end 163.00 67.50) (width 0.25) (layer "F.Cu") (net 19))
 (via (at 163.00 67.50) (size 0.80) (drill 0.40) (layers "F.Cu" "B.Cu") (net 19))
 (segment (start 163.00 67.50) (end 182.00 67.50) (width 0.25) (layer "B.Cu") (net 19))
 (segment (start 182.00 67.50) (end 182.00 66.16) (width 0.25) (layer "B.Cu") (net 19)))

